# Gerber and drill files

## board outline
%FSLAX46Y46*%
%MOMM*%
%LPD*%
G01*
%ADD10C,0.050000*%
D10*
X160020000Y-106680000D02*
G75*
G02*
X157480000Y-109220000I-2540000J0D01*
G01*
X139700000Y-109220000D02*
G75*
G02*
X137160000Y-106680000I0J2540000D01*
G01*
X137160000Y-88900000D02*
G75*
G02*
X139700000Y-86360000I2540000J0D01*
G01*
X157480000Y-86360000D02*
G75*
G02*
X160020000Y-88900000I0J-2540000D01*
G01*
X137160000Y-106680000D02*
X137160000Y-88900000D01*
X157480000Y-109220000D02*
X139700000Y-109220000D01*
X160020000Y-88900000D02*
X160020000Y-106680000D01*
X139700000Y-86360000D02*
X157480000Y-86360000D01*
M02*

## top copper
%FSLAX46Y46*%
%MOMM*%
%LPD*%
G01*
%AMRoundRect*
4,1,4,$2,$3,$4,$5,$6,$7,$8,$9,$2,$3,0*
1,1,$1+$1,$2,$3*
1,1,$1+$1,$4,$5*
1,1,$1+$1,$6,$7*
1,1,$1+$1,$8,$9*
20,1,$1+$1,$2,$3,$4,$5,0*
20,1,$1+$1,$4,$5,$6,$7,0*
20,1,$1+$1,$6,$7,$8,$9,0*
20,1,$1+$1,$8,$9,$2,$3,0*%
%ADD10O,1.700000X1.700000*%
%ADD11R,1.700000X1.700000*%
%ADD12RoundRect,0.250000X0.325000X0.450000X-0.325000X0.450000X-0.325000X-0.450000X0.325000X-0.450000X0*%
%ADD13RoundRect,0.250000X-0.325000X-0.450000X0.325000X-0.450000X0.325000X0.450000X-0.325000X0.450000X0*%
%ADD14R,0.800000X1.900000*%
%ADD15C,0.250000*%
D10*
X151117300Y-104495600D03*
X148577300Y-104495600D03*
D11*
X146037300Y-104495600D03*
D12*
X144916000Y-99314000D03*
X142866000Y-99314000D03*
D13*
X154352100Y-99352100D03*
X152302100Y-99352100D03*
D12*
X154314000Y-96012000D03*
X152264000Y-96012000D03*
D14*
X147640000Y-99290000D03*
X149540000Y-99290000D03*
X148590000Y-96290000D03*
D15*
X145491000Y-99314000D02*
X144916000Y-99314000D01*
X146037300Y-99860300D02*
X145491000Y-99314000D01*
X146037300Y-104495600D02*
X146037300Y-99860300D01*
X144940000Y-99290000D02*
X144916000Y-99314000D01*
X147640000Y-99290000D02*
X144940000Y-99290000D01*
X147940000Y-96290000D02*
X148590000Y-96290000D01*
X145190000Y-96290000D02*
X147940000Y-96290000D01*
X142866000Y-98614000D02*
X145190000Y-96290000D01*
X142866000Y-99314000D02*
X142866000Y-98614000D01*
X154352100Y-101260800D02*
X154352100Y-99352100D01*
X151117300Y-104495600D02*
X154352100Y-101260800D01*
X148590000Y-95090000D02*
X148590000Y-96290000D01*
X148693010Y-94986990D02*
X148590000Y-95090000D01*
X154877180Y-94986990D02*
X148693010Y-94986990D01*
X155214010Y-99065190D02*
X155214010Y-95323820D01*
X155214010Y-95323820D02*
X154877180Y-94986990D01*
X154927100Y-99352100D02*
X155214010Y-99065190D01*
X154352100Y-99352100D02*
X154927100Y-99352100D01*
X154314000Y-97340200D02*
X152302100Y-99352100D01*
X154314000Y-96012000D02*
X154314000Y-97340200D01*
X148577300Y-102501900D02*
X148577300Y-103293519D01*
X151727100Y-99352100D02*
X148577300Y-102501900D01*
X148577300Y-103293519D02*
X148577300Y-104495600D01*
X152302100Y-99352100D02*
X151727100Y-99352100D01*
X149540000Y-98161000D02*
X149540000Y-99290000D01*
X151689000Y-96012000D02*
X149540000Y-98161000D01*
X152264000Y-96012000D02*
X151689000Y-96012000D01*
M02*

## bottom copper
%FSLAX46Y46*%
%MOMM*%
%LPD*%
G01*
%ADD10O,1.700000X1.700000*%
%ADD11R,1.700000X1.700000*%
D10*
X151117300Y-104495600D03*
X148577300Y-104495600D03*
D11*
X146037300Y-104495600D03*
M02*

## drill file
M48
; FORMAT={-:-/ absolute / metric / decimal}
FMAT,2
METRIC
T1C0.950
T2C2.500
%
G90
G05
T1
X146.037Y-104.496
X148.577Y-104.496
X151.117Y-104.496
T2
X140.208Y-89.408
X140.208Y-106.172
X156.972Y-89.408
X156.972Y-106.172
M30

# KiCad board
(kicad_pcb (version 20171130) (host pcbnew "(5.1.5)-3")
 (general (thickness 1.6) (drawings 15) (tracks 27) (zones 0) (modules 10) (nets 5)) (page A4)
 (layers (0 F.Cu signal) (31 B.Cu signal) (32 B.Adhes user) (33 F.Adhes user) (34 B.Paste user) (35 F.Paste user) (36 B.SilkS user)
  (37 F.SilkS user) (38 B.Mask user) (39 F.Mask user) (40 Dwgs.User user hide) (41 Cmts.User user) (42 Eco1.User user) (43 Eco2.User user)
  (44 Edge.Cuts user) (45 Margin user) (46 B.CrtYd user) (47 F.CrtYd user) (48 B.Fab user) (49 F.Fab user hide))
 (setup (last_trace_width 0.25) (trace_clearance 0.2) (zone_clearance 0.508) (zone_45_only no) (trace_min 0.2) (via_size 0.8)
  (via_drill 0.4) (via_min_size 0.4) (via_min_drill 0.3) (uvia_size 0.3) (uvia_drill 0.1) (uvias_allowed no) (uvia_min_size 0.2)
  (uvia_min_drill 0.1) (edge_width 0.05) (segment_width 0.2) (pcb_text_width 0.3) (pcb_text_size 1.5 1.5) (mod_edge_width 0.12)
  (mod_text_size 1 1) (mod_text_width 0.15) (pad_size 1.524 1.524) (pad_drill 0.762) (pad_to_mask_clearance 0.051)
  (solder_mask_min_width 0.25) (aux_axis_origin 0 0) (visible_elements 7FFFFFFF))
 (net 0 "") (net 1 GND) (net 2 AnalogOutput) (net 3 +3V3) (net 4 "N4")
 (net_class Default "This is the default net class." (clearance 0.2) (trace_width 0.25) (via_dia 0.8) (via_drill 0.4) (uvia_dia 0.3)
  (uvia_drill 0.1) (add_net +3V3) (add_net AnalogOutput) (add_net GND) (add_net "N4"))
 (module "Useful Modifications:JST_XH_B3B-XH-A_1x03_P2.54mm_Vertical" (layer F.Cu) (at 146.0373 104.4956)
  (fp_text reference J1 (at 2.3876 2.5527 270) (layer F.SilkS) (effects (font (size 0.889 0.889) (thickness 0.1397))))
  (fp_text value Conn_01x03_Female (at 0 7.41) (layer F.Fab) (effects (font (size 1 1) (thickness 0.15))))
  (pad 3 thru_hole oval (at 5.08 0) (size 1.7 1.7) (drill 0.95) (layers *.Cu *.Mask) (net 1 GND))
  (pad 2 thru_hole oval (at 2.54 0) (size 1.7 1.7) (drill 0.95) (layers *.Cu *.Mask) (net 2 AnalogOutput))
  (pad 1 thru_hole rect (at 0 0) (size 1.7 1.7) (drill 0.95) (layers *.Cu *.Mask) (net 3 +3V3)))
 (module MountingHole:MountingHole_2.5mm (layer F.Cu) (at 140.208 89.408)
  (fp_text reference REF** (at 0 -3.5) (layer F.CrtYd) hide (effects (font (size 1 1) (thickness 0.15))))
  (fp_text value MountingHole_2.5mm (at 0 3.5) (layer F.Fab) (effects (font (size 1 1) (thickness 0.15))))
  (pad 1 np_thru_hole circle (at 0 0) (size 2.5 2.5) (drill 2.5) (layers *.Cu *.Mask)))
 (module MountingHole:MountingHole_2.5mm (layer F.Cu) (at 140.208 106.172)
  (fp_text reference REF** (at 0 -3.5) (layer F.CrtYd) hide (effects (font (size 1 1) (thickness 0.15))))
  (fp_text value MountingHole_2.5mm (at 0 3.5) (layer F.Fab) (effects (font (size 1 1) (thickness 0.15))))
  (pad 1 np_thru_hole circle (at 0 0) (size 2.5 2.5) (drill 2.5) (layers *.Cu *.Mask)))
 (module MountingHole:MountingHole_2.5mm (layer F.Cu) (at 156.972 106.172)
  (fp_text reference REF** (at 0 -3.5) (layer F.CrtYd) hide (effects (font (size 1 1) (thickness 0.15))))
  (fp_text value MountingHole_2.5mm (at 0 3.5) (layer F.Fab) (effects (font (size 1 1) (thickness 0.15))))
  (pad 1 np_thru_hole circle (at 0 0) (size 2.5 2.5) (drill 2.5) (layers *.Cu *.Mask)))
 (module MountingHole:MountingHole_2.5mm (layer F.Cu) (at 156.972 89.408)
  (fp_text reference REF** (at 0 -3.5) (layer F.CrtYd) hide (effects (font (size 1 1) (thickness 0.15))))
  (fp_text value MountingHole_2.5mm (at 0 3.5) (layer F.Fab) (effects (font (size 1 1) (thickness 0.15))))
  (pad 1 np_thru_hole circle (at 0 0) (size 2.5 2.5) (drill 2.5) (layers *.Cu *.Mask)))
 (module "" (layer F.Cu) (at 148.844 99.1108)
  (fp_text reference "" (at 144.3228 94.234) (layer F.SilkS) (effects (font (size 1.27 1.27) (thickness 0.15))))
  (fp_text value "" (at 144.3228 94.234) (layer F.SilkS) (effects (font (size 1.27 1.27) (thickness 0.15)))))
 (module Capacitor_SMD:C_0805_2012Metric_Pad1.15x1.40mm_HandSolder (layer F.Cu) (at 143.891 99.314 180)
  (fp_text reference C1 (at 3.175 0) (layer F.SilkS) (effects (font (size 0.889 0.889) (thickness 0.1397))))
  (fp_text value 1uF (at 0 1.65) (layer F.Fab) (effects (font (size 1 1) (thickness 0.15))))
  (pad 1 smd roundrect (at -1.025 0 180) (size 1.15 1.4) (layers F.Cu F.Paste F.Mask) (roundrect_rratio 0.217391) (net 3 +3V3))
  (pad 2 smd roundrect (at 1.025 0 180) (size 1.15 1.4) (layers F.Cu F.Paste F.Mask) (roundrect_rratio 0.217391) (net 1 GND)))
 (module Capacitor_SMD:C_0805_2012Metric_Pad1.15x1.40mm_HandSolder (layer F.Cu) (at 153.3271 99.3521)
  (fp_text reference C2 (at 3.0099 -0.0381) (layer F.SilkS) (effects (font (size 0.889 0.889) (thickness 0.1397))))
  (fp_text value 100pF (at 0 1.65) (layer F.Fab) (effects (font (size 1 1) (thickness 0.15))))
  (pad 2 smd roundrect (at 1.025 0) (size 1.15 1.4) (layers F.Cu F.Paste F.Mask) (roundrect_rratio 0.217391) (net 1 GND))
  (pad 1 smd roundrect (at -1.025 0) (size 1.15 1.4) (layers F.Cu F.Paste F.Mask) (roundrect_rratio 0.217391) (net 2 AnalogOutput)))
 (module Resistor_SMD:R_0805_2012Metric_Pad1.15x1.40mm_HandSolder (layer F.Cu) (at 153.289 96.012 180)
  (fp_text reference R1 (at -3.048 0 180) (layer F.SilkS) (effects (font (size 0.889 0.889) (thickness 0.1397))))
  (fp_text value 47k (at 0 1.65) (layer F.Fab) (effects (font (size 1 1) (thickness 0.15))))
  (pad 1 smd roundrect (at -1.025 0 180) (size 1.15 1.4) (layers F.Cu F.Paste F.Mask) (roundrect_rratio 0.217391) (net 2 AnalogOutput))
  (pad 2 smd roundrect (at 1.025 0 180) (size 1.15 1.4) (layers F.Cu F.Paste F.Mask) (roundrect_rratio 0.217391) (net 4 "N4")))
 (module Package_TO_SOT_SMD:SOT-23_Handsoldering (layer F.Cu) (at 148.59 97.79 90)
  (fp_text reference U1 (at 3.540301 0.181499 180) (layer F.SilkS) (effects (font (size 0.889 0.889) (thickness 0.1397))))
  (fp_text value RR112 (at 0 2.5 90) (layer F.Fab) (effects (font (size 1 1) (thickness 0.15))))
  (pad 1 smd rect (at -1.5 -0.95 90) (size 1.9 0.8) (layers F.Cu F.Paste F.Mask) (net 3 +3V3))
  (pad 2 smd rect (at -1.5 0.95 90) (size 1.9 0.8) (layers F.Cu F.Paste F.Mask) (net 4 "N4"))
  (pad 3 smd rect (at 1.5 0 90) (size 1.9 0.8) (layers F.Cu F.Paste F.Mask) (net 1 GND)))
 (gr_arc (start 157.48 106.68) (end 157.48 109.22) (angle -90) (layer Edge.Cuts) (width 0.05))
 (gr_arc (start 139.7 106.68) (end 137.16 106.68) (angle -90) (layer Edge.Cuts) (width 0.05))
 (gr_arc (start 139.7 88.9) (end 139.7 86.36) (angle -90) (layer Edge.Cuts) (width 0.05))
 (gr_arc (start 157.48 88.9) (end 160.02 88.9) (angle -90) (layer Edge.Cuts) (width 0.05))
 (gr_line (start 137.16 106.68) (end 137.16 88.9) (layer Edge.Cuts) (width 0.05))
 (gr_line (start 157.48 109.22) (end 139.7 109.22) (layer Edge.Cuts) (width 0.05))
 (gr_line (start 160.02 88.9) (end 160.02 106.68) (layer Edge.Cuts) (width 0.05))
 (gr_line (start 139.7 86.36) (end 157.48 86.36) (layer Edge.Cuts) (width 0.05))
 (segment (start 145.491 99.314) (end 144.916 99.314) (width 0.25) (layer F.Cu) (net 3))
 (segment (start 146.0373 99.8603) (end 145.491 99.314) (width 0.25) (layer F.Cu) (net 3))
 (segment (start 146.0373 104.4956) (end 146.0373 99.8603) (width 0.25) (layer F.Cu) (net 3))
 (segment (start 144.94 99.29) (end 144.916 99.314) (width 0.25) (layer F.Cu) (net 3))
 (segment (start 147.64 99.29) (end 144.94 99.29) (width 0.25) (layer F.Cu) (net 3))
 (segment (start 147.94 96.29) (end 148.59 96.29) (width 0.25) (layer F.Cu) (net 1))
 (segment (start 145.19 96.29) (end 147.94 96.29) (width 0.25) (layer F.Cu) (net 1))
 (segment (start 142.866 98.614) (end 145.19 96.29) (width 0.25) (layer F.Cu) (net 1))
 (segment (start 142.866 99.314) (end 142.866 98.614) (width 0.25) (layer F.Cu) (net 1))
 (segment (start 154.3521 101.2608) (end 154.3521 99.3521) (width 0.25) (layer F.Cu) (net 1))
 (segment (start 151.1173 104.4956) (end 154.3521 101.2608) (width 0.25) (layer F.Cu) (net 1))
 (segment (start 148.59 95.09) (end 148.59 96.29) (width 0.25) (layer F.Cu) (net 1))
 (segment (start 148.69301 94.98699) (end 148.59 95.09) (width 0.25) (layer F.Cu) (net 1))
 (segment (start 154.87718 94.98699) (end 148.69301 94.98699) (width 0.25) (layer F.Cu) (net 1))
 (segment (start 155.21401 99.06519) (end 155.21401 95.32382) (width 0.25) (layer F.Cu) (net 1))
 (segment (start 155.21401 95.32382) (end 154.87718 94.98699) (width 0.25) (layer F.Cu) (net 1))
 (segment (start 154.9271 99.3521) (end 155.21401 99.06519) (width 0.25) (layer F.Cu) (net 1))
 (segment (start 154.3521 99.3521) (end 154.9271 99.3521) (width 0.25) (layer F.Cu) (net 1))
 (segment (start 154.314 97.3402) (end 152.3021 99.3521) (width 0.25) (layer F.Cu) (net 2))
 (segment (start 154.314 96.012) (end 154.314 97.3402) (width 0.25) (layer F.Cu) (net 2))
 (segment (start 148.5773 102.5019) (end 148.5773 103.293519) (width 0.25) (layer F.Cu) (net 2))
 (segment (start 151.7271 99.3521) (end 148.5773 102.5019) (width 0.25) (layer F.Cu) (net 2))
 (segment (start 148.5773 103.293519) (end 148.5773 104.4956) (width 0.25) (layer F.Cu) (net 2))
 (segment (start 152.3021 99.3521) (end 151.7271 99.3521) (width 0.25) (layer F.Cu) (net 2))
 (segment (start 149.54 98.161) (end 149.54 99.29) (width 0.25) (layer F.Cu) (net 4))
 (segment (start 151.689 96.012) (end 149.54 98.161) (width 0.25) (layer F.Cu) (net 4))
 (segment (start 152.264 96.012) (end 151.689 96.012) (width 0.25) (layer F.Cu) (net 4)))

